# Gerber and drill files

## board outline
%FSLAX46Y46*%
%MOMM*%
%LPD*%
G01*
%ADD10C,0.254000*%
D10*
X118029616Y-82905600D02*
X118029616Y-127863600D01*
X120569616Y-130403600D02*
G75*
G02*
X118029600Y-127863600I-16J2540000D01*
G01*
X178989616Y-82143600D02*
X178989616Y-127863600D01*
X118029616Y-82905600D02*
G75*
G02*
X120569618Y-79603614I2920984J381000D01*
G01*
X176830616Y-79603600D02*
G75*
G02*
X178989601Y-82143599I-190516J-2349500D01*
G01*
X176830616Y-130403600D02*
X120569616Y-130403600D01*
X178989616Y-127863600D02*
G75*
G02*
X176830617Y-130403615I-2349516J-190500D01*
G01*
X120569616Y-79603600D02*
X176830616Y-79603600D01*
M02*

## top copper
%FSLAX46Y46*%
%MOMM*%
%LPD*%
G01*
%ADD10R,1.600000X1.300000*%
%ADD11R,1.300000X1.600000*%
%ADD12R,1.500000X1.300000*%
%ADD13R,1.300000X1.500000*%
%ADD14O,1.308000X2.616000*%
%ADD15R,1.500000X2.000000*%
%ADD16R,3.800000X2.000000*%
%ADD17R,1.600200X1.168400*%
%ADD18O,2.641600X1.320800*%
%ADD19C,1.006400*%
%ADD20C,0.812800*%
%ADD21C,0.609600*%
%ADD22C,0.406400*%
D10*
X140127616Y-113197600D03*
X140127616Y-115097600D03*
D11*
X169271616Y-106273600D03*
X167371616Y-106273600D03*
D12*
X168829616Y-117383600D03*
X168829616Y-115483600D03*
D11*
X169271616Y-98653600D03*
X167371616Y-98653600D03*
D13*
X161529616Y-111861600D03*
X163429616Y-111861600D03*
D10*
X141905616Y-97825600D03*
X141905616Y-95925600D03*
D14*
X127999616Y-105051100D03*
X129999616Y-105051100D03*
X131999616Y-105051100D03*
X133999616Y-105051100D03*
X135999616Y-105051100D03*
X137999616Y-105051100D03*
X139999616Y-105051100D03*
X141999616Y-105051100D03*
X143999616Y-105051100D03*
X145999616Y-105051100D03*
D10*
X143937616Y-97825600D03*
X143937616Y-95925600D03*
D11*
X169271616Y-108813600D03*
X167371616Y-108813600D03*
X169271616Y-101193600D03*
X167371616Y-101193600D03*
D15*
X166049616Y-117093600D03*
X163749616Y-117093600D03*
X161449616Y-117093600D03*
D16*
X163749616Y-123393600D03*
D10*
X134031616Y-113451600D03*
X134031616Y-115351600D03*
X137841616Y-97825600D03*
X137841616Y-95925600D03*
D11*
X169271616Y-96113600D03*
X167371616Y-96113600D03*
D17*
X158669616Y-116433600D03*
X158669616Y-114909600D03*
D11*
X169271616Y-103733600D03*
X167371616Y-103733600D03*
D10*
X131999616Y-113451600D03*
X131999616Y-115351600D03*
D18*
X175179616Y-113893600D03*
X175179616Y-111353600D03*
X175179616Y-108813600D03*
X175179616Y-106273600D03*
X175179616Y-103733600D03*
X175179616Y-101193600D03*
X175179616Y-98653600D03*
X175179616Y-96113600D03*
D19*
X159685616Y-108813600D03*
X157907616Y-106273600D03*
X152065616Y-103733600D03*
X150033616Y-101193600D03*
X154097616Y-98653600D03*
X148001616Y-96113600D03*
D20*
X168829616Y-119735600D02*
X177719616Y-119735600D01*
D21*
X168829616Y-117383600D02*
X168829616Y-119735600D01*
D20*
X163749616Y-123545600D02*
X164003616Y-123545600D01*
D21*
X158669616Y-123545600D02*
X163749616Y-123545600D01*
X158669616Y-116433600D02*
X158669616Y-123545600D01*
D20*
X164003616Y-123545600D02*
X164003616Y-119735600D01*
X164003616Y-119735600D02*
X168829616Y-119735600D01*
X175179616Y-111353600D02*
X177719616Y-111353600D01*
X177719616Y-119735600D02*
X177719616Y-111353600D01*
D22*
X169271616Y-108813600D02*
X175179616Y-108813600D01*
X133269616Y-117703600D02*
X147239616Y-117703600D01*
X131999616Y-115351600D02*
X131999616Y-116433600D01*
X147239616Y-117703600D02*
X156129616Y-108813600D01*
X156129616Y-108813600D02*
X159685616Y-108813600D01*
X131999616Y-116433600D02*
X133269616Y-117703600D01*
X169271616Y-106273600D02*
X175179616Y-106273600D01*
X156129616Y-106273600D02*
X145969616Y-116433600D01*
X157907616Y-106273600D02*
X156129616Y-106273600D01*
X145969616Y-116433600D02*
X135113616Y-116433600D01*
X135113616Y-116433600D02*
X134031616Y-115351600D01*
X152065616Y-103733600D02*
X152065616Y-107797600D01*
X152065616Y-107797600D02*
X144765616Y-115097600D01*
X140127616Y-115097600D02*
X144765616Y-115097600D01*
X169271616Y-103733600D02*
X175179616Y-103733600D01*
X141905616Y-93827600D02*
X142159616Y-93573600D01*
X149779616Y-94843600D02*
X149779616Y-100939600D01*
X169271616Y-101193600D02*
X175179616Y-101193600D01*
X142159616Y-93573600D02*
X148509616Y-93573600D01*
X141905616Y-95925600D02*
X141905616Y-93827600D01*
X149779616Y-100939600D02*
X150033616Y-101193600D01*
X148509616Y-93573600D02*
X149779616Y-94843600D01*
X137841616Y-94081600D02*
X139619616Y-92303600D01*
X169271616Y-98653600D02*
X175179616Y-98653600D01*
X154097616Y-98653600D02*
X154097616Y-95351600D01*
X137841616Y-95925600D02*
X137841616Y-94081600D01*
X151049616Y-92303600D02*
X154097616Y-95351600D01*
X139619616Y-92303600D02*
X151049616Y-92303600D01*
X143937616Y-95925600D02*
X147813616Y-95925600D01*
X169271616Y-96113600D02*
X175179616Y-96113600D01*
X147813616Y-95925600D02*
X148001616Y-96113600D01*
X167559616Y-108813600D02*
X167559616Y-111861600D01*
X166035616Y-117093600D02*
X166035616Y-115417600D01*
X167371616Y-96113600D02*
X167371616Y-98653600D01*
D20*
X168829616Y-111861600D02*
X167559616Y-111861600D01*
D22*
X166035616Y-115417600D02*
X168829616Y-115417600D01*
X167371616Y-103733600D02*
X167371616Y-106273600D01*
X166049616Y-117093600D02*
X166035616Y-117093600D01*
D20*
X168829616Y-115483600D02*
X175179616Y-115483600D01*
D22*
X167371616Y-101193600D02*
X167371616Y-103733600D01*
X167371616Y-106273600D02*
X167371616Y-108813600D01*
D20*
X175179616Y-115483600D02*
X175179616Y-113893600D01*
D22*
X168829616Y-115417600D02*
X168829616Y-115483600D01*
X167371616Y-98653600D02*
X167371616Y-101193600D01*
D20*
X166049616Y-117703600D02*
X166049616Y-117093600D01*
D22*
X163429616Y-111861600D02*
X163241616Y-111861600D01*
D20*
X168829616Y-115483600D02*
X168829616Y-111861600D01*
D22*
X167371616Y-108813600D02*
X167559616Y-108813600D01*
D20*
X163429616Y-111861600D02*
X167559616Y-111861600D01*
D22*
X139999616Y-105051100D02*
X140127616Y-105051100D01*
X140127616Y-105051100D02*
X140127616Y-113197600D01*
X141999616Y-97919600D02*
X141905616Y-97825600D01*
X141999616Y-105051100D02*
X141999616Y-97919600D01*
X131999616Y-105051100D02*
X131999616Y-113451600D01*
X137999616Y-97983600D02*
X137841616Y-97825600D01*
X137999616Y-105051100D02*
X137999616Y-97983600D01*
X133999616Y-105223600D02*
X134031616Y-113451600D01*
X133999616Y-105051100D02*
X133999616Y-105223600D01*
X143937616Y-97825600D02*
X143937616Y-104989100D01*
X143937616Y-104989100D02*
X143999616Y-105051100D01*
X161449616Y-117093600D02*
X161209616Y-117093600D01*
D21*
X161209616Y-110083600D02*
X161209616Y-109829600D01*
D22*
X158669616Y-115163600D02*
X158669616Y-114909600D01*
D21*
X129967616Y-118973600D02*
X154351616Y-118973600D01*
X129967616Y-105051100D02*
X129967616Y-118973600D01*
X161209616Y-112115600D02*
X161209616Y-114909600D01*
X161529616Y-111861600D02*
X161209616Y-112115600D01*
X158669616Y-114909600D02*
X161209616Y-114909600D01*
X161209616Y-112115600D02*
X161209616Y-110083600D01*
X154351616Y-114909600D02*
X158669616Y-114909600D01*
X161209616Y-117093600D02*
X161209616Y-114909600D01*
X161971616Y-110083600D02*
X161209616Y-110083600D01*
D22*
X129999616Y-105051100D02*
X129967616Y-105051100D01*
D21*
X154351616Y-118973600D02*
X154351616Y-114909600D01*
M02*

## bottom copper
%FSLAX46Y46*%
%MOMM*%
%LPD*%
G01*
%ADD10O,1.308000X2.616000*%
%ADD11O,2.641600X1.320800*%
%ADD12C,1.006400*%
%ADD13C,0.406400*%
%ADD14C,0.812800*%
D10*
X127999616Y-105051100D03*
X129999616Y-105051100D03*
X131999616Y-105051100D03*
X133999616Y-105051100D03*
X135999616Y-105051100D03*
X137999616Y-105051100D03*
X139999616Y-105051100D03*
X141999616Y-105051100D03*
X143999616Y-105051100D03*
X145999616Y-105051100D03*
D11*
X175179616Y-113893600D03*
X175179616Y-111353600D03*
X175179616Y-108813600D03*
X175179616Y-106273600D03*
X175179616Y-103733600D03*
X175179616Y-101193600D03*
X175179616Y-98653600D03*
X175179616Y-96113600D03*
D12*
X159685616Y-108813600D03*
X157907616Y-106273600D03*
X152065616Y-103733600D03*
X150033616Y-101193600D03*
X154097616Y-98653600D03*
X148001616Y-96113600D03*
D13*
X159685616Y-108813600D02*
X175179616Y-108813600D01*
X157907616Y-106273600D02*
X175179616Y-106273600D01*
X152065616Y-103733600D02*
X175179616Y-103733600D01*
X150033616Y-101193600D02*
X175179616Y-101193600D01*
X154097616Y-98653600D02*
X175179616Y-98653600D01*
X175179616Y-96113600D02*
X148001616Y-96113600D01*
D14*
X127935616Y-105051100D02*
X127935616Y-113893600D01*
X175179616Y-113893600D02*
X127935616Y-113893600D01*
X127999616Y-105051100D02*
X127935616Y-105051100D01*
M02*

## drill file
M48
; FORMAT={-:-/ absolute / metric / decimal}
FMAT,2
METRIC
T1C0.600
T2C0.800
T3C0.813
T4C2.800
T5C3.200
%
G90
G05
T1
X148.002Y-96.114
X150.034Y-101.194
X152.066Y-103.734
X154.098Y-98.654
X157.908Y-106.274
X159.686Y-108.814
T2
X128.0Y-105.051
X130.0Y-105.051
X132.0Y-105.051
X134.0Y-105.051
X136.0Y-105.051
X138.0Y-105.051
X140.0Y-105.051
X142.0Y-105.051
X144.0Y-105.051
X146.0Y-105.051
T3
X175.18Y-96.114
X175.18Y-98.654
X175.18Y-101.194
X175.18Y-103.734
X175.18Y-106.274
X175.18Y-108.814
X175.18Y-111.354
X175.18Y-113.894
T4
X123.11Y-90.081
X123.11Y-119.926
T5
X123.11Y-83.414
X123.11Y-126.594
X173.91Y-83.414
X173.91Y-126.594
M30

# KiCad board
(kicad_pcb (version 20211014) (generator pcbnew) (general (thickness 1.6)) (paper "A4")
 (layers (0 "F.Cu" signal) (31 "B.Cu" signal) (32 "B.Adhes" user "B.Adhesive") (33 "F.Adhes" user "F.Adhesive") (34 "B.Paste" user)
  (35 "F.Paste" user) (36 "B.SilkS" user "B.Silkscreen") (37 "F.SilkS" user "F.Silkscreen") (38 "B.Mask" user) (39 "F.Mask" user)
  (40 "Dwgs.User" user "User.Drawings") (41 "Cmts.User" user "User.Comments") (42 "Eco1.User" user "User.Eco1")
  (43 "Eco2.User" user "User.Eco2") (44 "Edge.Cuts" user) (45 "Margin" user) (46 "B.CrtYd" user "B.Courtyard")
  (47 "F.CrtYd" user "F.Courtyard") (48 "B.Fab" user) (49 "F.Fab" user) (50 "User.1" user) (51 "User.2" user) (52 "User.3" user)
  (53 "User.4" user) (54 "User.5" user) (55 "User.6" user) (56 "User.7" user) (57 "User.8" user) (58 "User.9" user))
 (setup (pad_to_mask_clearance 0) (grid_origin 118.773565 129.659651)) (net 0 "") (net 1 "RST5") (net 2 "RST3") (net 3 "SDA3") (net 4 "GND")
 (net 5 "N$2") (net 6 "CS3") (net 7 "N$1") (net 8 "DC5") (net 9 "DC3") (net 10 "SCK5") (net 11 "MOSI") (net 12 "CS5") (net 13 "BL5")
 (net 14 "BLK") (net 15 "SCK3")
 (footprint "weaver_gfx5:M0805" (layer "F.Cu") (at 140.127616 114.1476 -90)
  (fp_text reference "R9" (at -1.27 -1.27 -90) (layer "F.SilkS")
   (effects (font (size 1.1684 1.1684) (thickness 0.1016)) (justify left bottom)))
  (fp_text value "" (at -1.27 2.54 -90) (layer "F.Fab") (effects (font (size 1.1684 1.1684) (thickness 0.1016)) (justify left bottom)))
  (pad "1" smd rect (at -0.95 0 270) (size 1.3 1.6) (layers "F.Cu" "F.Paste" "F.Mask") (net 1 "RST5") (solder_mask_margin 0.1016))
  (pad "2" smd rect (at 0.95 0 270) (size 1.3 1.6) (layers "F.Cu" "F.Paste" "F.Mask") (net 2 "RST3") (solder_mask_margin 0.1016)))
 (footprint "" (layer "F.Cu") (at 173.909616 83.4136)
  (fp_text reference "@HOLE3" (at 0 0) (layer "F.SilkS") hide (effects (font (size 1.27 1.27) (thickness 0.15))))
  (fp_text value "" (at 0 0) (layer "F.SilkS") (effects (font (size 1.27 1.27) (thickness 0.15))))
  (pad "" np_thru_hole circle (at 0 0) (size 3.2 3.2) (drill 3.2) (layers *.Cu *.Mask)))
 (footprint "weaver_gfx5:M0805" (layer "F.Cu") (at 168.321616 106.2736 180)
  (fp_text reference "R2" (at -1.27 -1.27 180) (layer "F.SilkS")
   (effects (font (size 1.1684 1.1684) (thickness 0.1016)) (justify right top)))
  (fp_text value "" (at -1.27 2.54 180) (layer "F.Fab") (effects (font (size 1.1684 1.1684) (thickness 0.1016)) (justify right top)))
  (pad "1" smd rect (at -0.95 0 180) (size 1.3 1.6) (layers "F.Cu" "F.Paste" "F.Mask") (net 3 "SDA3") (solder_mask_margin 0.1016))
  (pad "2" smd rect (at 0.95 0 180) (size 1.3 1.6) (layers "F.Cu" "F.Paste" "F.Mask") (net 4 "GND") (solder_mask_margin 0.1016)))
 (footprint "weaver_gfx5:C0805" (layer "F.Cu") (at 168.829616 116.4336 90)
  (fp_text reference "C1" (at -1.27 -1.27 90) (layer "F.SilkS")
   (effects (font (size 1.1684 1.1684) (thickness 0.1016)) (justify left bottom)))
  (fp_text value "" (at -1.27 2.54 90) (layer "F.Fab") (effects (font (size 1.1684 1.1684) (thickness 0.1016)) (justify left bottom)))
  (pad "1" smd rect (at -0.95 0 90) (size 1.3 1.5) (layers "F.Cu" "F.Paste" "F.Mask") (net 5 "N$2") (solder_mask_margin 0.1016))
  (pad "2" smd rect (at 0.95 0 90) (size 1.3 1.5) (layers "F.Cu" "F.Paste" "F.Mask") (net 4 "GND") (solder_mask_margin 0.1016)))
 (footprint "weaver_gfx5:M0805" (layer "F.Cu") (at 168.321616 98.6536 180)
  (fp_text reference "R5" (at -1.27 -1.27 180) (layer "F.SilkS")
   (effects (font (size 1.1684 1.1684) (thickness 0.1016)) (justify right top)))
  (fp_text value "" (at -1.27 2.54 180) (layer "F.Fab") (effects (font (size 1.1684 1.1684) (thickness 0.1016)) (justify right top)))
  (pad "1" smd rect (at -0.95 0 180) (size 1.3 1.6) (layers "F.Cu" "F.Paste" "F.Mask") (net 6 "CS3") (solder_mask_margin 0.1016))
  (pad "2" smd rect (at 0.95 0 180) (size 1.3 1.6) (layers "F.Cu" "F.Paste" "F.Mask") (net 4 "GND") (solder_mask_margin 0.1016)))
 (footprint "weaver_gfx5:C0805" (layer "F.Cu") (at 162.479616 111.8616)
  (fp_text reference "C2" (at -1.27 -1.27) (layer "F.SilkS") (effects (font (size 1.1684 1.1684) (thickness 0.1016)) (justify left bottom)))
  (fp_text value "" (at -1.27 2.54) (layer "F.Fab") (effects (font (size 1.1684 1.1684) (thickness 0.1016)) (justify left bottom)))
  (pad "1" smd rect (at -0.95 0) (size 1.3 1.5) (layers "F.Cu" "F.Paste" "F.Mask") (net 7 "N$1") (solder_mask_margin 0.1016))
  (pad "2" smd rect (at 0.95 0) (size 1.3 1.5) (layers "F.Cu" "F.Paste" "F.Mask") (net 4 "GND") (solder_mask_margin 0.1016)))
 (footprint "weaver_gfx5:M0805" (layer "F.Cu") (at 141.905616 96.8756 90)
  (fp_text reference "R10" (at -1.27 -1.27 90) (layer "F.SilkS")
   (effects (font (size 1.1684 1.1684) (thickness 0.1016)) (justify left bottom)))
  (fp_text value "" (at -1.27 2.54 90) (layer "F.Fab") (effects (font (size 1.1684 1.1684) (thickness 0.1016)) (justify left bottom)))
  (pad "1" smd rect (at -0.95 0 90) (size 1.3 1.6) (layers "F.Cu" "F.Paste" "F.Mask") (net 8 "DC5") (solder_mask_margin 0.1016))
  (pad "2" smd rect (at 0.95 0 90) (size 1.3 1.6) (layers "F.Cu" "F.Paste" "F.Mask") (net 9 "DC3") (solder_mask_margin 0.1016)))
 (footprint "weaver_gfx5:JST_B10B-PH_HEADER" (layer "F.Cu") (at 131.999616 105.0036 180)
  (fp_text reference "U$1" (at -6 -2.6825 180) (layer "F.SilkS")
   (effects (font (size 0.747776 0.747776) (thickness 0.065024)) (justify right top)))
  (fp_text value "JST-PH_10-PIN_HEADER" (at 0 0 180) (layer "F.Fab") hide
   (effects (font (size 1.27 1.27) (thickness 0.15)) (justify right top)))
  (pad "P1" thru_hole oval (at 4 -0.0475 270) (size 2.616 1.308) (drill 0.8) (layers *.Cu *.Mask) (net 4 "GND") (solder_mask_margin 0.1016))
  (pad "P2" thru_hole oval (at 2 -0.0475 270) (size 2.616 1.308) (drill 0.8) (layers *.Cu *.Mask) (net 7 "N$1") (solder_mask_margin 0.1016))
  (pad "P3" thru_hole oval (at 0 -0.0475 270) (size 2.616 1.308) (drill 0.8) (layers *.Cu *.Mask) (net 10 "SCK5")
   (solder_mask_margin 0.1016))
  (pad "P4" thru_hole oval (at -2 -0.0475 270) (size 2.616 1.308) (drill 0.8) (layers *.Cu *.Mask) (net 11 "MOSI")
   (solder_mask_margin 0.1016))
  (pad "P5" thru_hole oval (at -4 -0.0475 270) (size 2.616 1.308) (drill 0.8) (layers *.Cu *.Mask) (solder_mask_margin 0.1016))
  (pad "P6" thru_hole oval (at -6 -0.0475 270) (size 2.616 1.308) (drill 0.8) (layers *.Cu *.Mask) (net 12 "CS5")
   (solder_mask_margin 0.1016))
  (pad "P7" thru_hole oval (at -8 -0.0475 270) (size 2.616 1.308) (drill 0.8) (layers *.Cu *.Mask) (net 1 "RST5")
   (solder_mask_margin 0.1016))
  (pad "P8" thru_hole oval (at -10 -0.0475 270) (size 2.616 1.308) (drill 0.8) (layers *.Cu *.Mask) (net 8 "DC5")
   (solder_mask_margin 0.1016))
  (pad "P9" thru_hole oval (at -12 -0.0475 270) (size 2.616 1.308) (drill 0.8) (layers *.Cu *.Mask) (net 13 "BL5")
   (solder_mask_margin 0.1016))
  (pad "P10" thru_hole oval (at -14 -0.0475 270) (size 2.616 1.308) (drill 0.8) (layers *.Cu *.Mask) (solder_mask_margin 0.1016)))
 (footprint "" (layer "F.Cu") (at 123.109616 83.4136)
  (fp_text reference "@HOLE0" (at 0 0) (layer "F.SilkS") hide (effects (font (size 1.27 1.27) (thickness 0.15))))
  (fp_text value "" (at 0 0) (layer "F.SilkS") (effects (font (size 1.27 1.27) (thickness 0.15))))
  (pad "" np_thru_hole circle (at 0 0) (size 3.2 3.2) (drill 3.2) (layers *.Cu *.Mask)))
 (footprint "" (layer "F.Cu") (at 123.109616 90.0811)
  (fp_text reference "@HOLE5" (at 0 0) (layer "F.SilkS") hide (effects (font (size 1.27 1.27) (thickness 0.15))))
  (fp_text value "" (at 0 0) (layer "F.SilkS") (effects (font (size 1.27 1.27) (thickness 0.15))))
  (pad "" np_thru_hole circle (at 0 0) (size 2.8 2.8) (drill 2.8) (layers *.Cu *.Mask)))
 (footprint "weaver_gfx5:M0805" (layer "F.Cu") (at 143.937616 96.8756 90)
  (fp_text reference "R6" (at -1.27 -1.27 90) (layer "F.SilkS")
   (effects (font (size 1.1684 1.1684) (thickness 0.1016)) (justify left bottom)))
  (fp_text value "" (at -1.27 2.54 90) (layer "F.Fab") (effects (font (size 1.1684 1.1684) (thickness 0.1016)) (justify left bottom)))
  (pad "1" smd rect (at -0.95 0 90) (size 1.3 1.6) (layers "F.Cu" "F.Paste" "F.Mask") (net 13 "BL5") (solder_mask_margin 0.1016))
  (pad "2" smd rect (at 0.95 0 90) (size 1.3 1.6) (layers "F.Cu" "F.Paste" "F.Mask") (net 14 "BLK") (solder_mask_margin 0.1016)))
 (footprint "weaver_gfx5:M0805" (layer "F.Cu") (at 168.321616 108.8136 180)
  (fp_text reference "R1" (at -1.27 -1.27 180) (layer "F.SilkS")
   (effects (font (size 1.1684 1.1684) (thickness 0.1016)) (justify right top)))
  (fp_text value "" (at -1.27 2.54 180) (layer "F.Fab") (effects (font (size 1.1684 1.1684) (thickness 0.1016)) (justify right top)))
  (pad "1" smd rect (at -0.95 0 180) (size 1.3 1.6) (layers "F.Cu" "F.Paste" "F.Mask") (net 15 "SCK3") (solder_mask_margin 0.1016))
  (pad "2" smd rect (at 0.95 0 180) (size 1.3 1.6) (layers "F.Cu" "F.Paste" "F.Mask") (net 4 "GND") (solder_mask_margin 0.1016)))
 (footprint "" (layer "F.Cu") (at 123.109616 119.9261)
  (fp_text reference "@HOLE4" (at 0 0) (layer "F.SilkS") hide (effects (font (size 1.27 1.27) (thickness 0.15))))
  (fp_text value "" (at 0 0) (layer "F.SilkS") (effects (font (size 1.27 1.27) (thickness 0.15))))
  (pad "" np_thru_hole circle (at 0 0) (size 2.8 2.8) (drill 2.8) (layers *.Cu *.Mask)))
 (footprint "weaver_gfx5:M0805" (layer "F.Cu") (at 168.321616 101.1936 180)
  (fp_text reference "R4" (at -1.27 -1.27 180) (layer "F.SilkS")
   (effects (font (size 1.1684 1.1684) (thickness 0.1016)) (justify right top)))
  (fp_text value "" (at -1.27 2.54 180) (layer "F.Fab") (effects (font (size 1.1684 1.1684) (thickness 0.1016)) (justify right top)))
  (pad "1" smd rect (at -0.95 0 180) (size 1.3 1.6) (layers "F.Cu" "F.Paste" "F.Mask") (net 9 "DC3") (solder_mask_margin 0.1016))
  (pad "2" smd rect (at 0.95 0 180) (size 1.3 1.6) (layers "F.Cu" "F.Paste" "F.Mask") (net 4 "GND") (solder_mask_margin 0.1016)))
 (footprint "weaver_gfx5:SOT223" (layer "F.Cu") (at 163.749616 120.2436 180)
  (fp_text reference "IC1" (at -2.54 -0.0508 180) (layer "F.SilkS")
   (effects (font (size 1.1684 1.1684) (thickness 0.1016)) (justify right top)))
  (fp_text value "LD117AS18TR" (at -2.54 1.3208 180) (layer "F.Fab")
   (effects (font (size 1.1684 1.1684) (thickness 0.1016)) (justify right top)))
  (pad "1" smd rect (at -2.3 3.15 180) (size 1.5 2) (layers "F.Cu" "F.Paste" "F.Mask") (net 4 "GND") (solder_mask_margin 0.1016))
  (pad "2" smd rect (at 0 3.15 180) (size 1.5 2) (layers "F.Cu" "F.Paste" "F.Mask") (solder_mask_margin 0.1016))
  (pad "3" smd rect (at 2.3 3.15 180) (size 1.5 2) (layers "F.Cu" "F.Paste" "F.Mask") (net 7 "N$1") (solder_mask_margin 0.1016))
  (pad "4" smd rect (at 0 -3.15 180) (size 3.8 2) (layers "F.Cu" "F.Paste" "F.Mask") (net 5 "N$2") (solder_mask_margin 0.1016)))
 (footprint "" (layer "F.Cu") (at 123.109616 126.5936)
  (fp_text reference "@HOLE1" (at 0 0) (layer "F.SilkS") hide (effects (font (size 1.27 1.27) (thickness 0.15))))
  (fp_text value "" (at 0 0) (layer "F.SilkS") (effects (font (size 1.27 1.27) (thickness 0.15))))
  (pad "" np_thru_hole circle (at 0 0) (size 3.2 3.2) (drill 3.2) (layers *.Cu *.Mask)))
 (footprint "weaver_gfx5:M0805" (layer "F.Cu") (at 134.031616 114.4016 -90)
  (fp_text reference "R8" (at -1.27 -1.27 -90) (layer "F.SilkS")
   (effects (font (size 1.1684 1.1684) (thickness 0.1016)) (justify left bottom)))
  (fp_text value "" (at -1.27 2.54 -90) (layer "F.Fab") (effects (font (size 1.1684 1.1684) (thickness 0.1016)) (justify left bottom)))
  (pad "1" smd rect (at -0.95 0 270) (size 1.3 1.6) (layers "F.Cu" "F.Paste" "F.Mask") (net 11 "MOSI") (solder_mask_margin 0.1016))
  (pad "2" smd rect (at 0.95 0 270) (size 1.3 1.6) (layers "F.Cu" "F.Paste" "F.Mask") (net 3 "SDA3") (solder_mask_margin 0.1016)))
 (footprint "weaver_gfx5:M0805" (layer "F.Cu") (at 137.841616 96.8756 90)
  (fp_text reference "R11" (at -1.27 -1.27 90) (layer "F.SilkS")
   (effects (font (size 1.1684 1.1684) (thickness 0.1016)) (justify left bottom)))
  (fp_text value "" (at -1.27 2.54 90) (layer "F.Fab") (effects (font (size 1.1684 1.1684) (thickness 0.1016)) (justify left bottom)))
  (pad "1" smd rect (at -0.95 0 90) (size 1.3 1.6) (layers "F.Cu" "F.Paste" "F.Mask") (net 12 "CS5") (solder_mask_margin 0.1016))
  (pad "2" smd rect (at 0.95 0 90) (size 1.3 1.6) (layers "F.Cu" "F.Paste" "F.Mask") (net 6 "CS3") (solder_mask_margin 0.1016)))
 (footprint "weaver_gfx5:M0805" (layer "F.Cu") (at 168.321616 96.1136 180)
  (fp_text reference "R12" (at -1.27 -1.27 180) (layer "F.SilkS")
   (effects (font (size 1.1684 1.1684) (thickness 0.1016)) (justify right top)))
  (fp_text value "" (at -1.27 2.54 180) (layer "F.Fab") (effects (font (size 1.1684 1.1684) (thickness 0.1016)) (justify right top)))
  (pad "1" smd rect (at -0.95 0 180) (size 1.3 1.6) (layers "F.Cu" "F.Paste" "F.Mask") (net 14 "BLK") (solder_mask_margin 0.1016))
  (pad "2" smd rect (at 0.95 0 180) (size 1.3 1.6) (layers "F.Cu" "F.Paste" "F.Mask") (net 4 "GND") (solder_mask_margin 0.1016)))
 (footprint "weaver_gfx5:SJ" (layer "F.Cu") (at 158.669616 115.6716 90)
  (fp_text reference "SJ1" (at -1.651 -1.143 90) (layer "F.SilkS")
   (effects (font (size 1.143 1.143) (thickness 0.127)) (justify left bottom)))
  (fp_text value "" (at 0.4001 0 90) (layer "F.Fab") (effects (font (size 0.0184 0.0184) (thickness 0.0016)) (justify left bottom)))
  (pad "1" smd rect (at -0.762 0 90) (size 1.1684 1.6002) (layers "F.Cu" "F.Paste" "F.Mask") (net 5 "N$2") (solder_mask_margin 0.1016))
  (pad "2" smd rect (at 0.762 0 90) (size 1.1684 1.6002) (layers "F.Cu" "F.Paste" "F.Mask") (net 7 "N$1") (solder_mask_margin 0.1016)))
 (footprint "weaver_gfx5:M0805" (layer "F.Cu") (at 168.321616 103.7336 180)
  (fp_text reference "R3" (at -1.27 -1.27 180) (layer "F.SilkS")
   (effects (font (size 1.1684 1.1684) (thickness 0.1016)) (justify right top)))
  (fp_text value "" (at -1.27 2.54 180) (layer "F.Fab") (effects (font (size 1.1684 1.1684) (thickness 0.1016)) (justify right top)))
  (pad "1" smd rect (at -0.95 0 180) (size 1.3 1.6) (layers "F.Cu" "F.Paste" "F.Mask") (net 2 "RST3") (solder_mask_margin 0.1016))
  (pad "2" smd rect (at 0.95 0 180) (size 1.3 1.6) (layers "F.Cu" "F.Paste" "F.Mask") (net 4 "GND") (solder_mask_margin 0.1016)))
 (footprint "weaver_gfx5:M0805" (layer "F.Cu") (at 131.999616 114.4016 -90)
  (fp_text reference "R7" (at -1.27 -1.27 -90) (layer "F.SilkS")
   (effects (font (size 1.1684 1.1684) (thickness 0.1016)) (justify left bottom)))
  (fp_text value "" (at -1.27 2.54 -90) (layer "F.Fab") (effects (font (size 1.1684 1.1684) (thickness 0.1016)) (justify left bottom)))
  (pad "1" smd rect (at -0.95 0 270) (size 1.3 1.6) (layers "F.Cu" "F.Paste" "F.Mask") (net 10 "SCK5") (solder_mask_margin 0.1016))
  (pad "2" smd rect (at 0.95 0 270) (size 1.3 1.6) (layers "F.Cu" "F.Paste" "F.Mask") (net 15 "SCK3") (solder_mask_margin 0.1016)))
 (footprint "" (layer "F.Cu") (at 173.909616 126.5936)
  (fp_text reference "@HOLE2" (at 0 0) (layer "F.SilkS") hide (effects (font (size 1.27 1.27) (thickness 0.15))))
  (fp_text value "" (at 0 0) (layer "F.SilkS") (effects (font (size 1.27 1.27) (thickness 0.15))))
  (pad "" np_thru_hole circle (at 0 0) (size 3.2 3.2) (drill 3.2) (layers *.Cu *.Mask)))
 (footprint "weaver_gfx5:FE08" (layer "B.Cu") (at 175.179616 105.0036 90)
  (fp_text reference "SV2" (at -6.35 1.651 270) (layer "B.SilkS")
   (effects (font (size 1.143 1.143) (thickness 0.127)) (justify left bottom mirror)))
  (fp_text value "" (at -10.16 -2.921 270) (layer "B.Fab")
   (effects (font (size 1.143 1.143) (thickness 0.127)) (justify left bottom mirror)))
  (pad "1" thru_hole oval (at -8.89 0) (size 2.6416 1.3208) (drill 0.8128) (layers *.Cu *.Mask) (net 4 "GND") (solder_mask_margin 0.1016))
  (pad "2" thru_hole oval (at -6.35 0) (size 2.6416 1.3208) (drill 0.8128) (layers *.Cu *.Mask) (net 5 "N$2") (solder_mask_margin 0.1016))
  (pad "3" thru_hole oval (at -3.81 0) (size 2.6416 1.3208) (drill 0.8128) (layers *.Cu *.Mask) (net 15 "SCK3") (solder_mask_margin 0.1016))
  (pad "4" thru_hole oval (at -1.27 0) (size 2.6416 1.3208) (drill 0.8128) (layers *.Cu *.Mask) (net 3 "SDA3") (solder_mask_margin 0.1016))
  (pad "5" thru_hole oval (at 1.27 0) (size 2.6416 1.3208) (drill 0.8128) (layers *.Cu *.Mask) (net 2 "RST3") (solder_mask_margin 0.1016))
  (pad "6" thru_hole oval (at 3.81 0) (size 2.6416 1.3208) (drill 0.8128) (layers *.Cu *.Mask) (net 9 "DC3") (solder_mask_margin 0.1016))
  (pad "7" thru_hole oval (at 6.35 0) (size 2.6416 1.3208) (drill 0.8128) (layers *.Cu *.Mask) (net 6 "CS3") (solder_mask_margin 0.1016))
  (pad "8" thru_hole oval (at 8.89 0) (size 2.6416 1.3208) (drill 0.8128) (layers *.Cu *.Mask) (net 14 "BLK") (solder_mask_margin 0.1016)))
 (gr_line (start 118.029616 82.9056) (end 118.029616 127.8636) (layer "Edge.Cuts") (width 0.254))
 (gr_arc (start 120.569616 130.4036) (mid 118.773565 129.659651) (end 118.029616 127.8636) (layer "Edge.Cuts") (width 0.254))
 (gr_line (start 178.989616 82.1436) (end 178.989616 127.8636) (layer "Edge.Cuts") (width 0.254))
 (gr_arc (start 118.029616 82.9056) (mid 118.615749 80.728549) (end 120.569616 79.6036) (layer "Edge.Cuts") (width 0.254))
 (gr_arc (start 176.830616 79.6036) (mid 178.436167 80.426456) (end 178.989616 82.1436) (layer "Edge.Cuts") (width 0.254))
 (gr_line (start 176.830616 130.4036) (end 120.569616 130.4036) (layer "Edge.Cuts") (width 0.254))
 (gr_arc (start 178.989616 127.8636) (mid 178.436167 129.580744) (end 176.830616 130.4036) (layer "Edge.Cuts") (width 0.254))
 (gr_line (start 120.569616 79.6036) (end 176.830616 79.6036) (layer "Edge.Cuts") (width 0.254))
 (segment (start 168.829616 119.7356) (end 177.719616 119.7356) (width 0.8128) (layer "F.Cu") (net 5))
 (segment (start 168.829616 117.3836) (end 168.829616 119.7356) (width 0.6096) (layer "F.Cu") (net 5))
 (segment (start 163.749616 123.5456) (end 164.003616 123.5456) (width 0.8128) (layer "F.Cu") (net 5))
 (segment (start 158.669616 123.5456) (end 163.749616 123.5456) (width 0.6096) (layer "F.Cu") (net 5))
 (segment (start 158.669616 116.4336) (end 158.669616 123.5456) (width 0.6096) (layer "F.Cu") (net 5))
 (segment (start 164.003616 123.5456) (end 164.003616 119.7356) (width 0.8128) (layer "F.Cu") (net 5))
 (segment (start 164.003616 119.7356) (end 168.829616 119.7356) (width 0.8128) (layer "F.Cu") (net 5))
 (segment (start 175.179616 111.3536) (end 177.719616 111.3536) (width 0.8128) (layer "F.Cu") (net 5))
 (segment (start 177.719616 119.7356) (end 177.719616 111.3536) (width 0.8128) (layer "F.Cu") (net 5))
 (segment (start 169.271616 108.8136) (end 175.179616 108.8136) (width 0.4064) (layer "F.Cu") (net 15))
 (segment (start 133.269616 117.7036) (end 147.239616 117.7036) (width 0.4064) (layer "F.Cu") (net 15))
 (segment (start 131.999616 115.3516) (end 131.999616 116.4336) (width 0.4064) (layer "F.Cu") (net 15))
 (segment (start 147.239616 117.7036) (end 156.129616 108.8136) (width 0.4064) (layer "F.Cu") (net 15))
 (segment (start 156.129616 108.8136) (end 159.685616 108.8136) (width 0.4064) (layer "F.Cu") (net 15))
 (segment (start 131.999616 116.4336) (end 133.269616 117.7036) (width 0.4064) (layer "F.Cu") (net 15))
 (via (at 159.685616 108.8136) (size 1.0064) (drill 0.6) (layers "F.Cu" "B.Cu") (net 15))
 (segment (start 159.685616 108.8136) (end 175.179616 108.8136) (width 0.4064) (layer "B.Cu") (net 15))
 (segment (start 169.271616 106.2736) (end 175.179616 106.2736) (width 0.4064) (layer "F.Cu") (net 3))
 (segment (start 156.129616 106.2736) (end 145.969616 116.4336) (width 0.4064) (layer "F.Cu") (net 3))
 (segment (start 157.907616 106.2736) (end 156.129616 106.2736) (width 0.4064) (layer "F.Cu") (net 3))
 (segment (start 145.969616 116.4336) (end 135.113616 116.4336) (width 0.4064) (layer "F.Cu") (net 3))
 (segment (start 135.113616 116.4336) (end 134.031616 115.3516) (width 0.4064) (layer "F.Cu") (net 3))
 (via (at 157.907616 106.2736) (size 1.0064) (drill 0.6) (layers "F.Cu" "B.Cu") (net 3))
 (segment (start 157.907616 106.2736) (end 175.179616 106.2736) (width 0.4064) (layer "B.Cu") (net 3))
 (segment (start 152.065616 103.7336) (end 152.065616 107.7976) (width 0.4064) (layer "F.Cu") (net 2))
 (segment (start 152.065616 107.7976) (end 144.765616 115.0976) (width 0.4064) (layer "F.Cu") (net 2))
 (segment (start 140.127616 115.0976) (end 144.765616 115.0976) (width 0.4064) (layer "F.Cu") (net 2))
 (segment (start 169.271616 103.7336) (end 175.179616 103.7336) (width 0.4064) (layer "F.Cu") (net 2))
 (via (at 152.065616 103.7336) (size 1.0064) (drill 0.6) (layers "F.Cu" "B.Cu") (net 2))
 (segment (start 152.065616 103.7336) (end 175.179616 103.7336) (width 0.4064) (layer "B.Cu") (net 2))
 (segment (start 141.905616 93.8276) (end 142.159616 93.5736) (width 0.4064) (layer "F.Cu") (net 9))
 (segment (start 149.779616 94.8436) (end 149.779616 100.9396) (width 0.4064) (layer "F.Cu") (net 9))
 (segment (start 169.271616 101.1936) (end 175.179616 101.1936) (width 0.4064) (layer "F.Cu") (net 9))
 (segment (start 142.159616 93.5736) (end 148.509616 93.5736) (width 0.4064) (layer "F.Cu") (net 9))
 (segment (start 141.905616 95.9256) (end 141.905616 93.8276) (width 0.4064) (layer "F.Cu") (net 9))
 (segment (start 149.779616 100.9396) (end 150.033616 101.1936) (width 0.4064) (layer "F.Cu") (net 9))
 (segment (start 148.509616 93.5736) (end 149.779616 94.8436) (width 0.4064) (layer "F.Cu") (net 9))
 (via (at 150.033616 101.1936) (size 1.0064) (drill 0.6) (layers "F.Cu" "B.Cu") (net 9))
 (segment (start 150.033616 101.1936) (end 175.179616 101.1936) (width 0.4064) (layer "B.Cu") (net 9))
 (segment (start 137.841616 94.0816) (end 139.619616 92.3036) (width 0.4064) (layer "F.Cu") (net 6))
 (segment (start 169.271616 98.6536) (end 175.179616 98.6536) (width 0.4064) (layer "F.Cu") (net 6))
 (segment (start 154.097616 98.6536) (end 154.097616 95.3516) (width 0.4064) (layer "F.Cu") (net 6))
 (segment (start 137.841616 95.9256) (end 137.841616 94.0816) (width 0.4064) (layer "F.Cu") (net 6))
 (segment (start 151.049616 92.3036) (end 154.097616 95.3516) (width 0.4064) (layer "F.Cu") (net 6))
 (segment (start 139.619616 92.3036) (end 151.049616 92.3036) (width 0.4064) (layer "F.Cu") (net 6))
 (via (at 154.097616 98.6536) (size 1.0064) (drill 0.6) (layers "F.Cu" "B.Cu") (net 6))
 (segment (start 154.097616 98.6536) (end 175.179616 98.6536) (width 0.4064) (layer "B.Cu") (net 6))
 (segment (start 143.937616 95.9256) (end 147.813616 95.9256) (width 0.4064) (layer "F.Cu") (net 14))
 (segment (start 169.271616 96.1136) (end 175.179616 96.1136) (width 0.4064) (layer "F.Cu") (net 14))
 (segment (start 147.813616 95.9256) (end 148.001616 96.1136) (width 0.4064) (layer "F.Cu") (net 14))
 (via (at 148.001616 96.1136) (size 1.0064) (drill 0.6) (layers "F.Cu" "B.Cu") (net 14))
 (segment (start 175.179616 96.1136) (end 148.001616 96.1136) (width 0.4064) (layer "B.Cu") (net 14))
 (segment (start 167.559616 108.8136) (end 167.559616 111.8616) (width 0.4064) (layer "F.Cu") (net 4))
 (segment (start 166.035616 117.0936) (end 166.035616 115.4176) (width 0.4064) (layer "F.Cu") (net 4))
 (segment (start 167.371616 96.1136) (end 167.371616 98.6536) (width 0.4064) (layer "F.Cu") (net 4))
 (segment (start 168.829616 111.8616) (end 167.559616 111.8616) (width 0.8128) (layer "F.Cu") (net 4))
 (segment (start 166.035616 115.4176) (end 168.829616 115.4176) (width 0.4064) (layer "F.Cu") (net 4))
 (segment (start 167.371616 103.7336) (end 167.371616 106.2736) (width 0.4064) (layer "F.Cu") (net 4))
 (segment (start 166.049616 117.0936) (end 166.035616 117.0936) (width 0.4064) (layer "F.Cu") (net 4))
 (segment (start 168.829616 115.4836) (end 175.179616 115.4836) (width 0.8128) (layer "F.Cu") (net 4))
 (segment (start 167.371616 101.1936) (end 167.371616 103.7336) (width 0.4064) (layer "F.Cu") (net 4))
 (segment (start 167.371616 106.2736) (end 167.371616 108.8136) (width 0.4064) (layer "F.Cu") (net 4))
 (segment (start 175.179616 115.4836) (end 175.179616 113.8936) (width 0.8128) (layer "F.Cu") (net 4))
 (segment (start 168.829616 115.4176) (end 168.829616 115.4836) (width 0.4064) (layer "F.Cu") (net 4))
 (segment (start 167.371616 98.6536) (end 167.371616 101.1936) (width 0.4064) (layer "F.Cu") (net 4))
 (segment (start 166.049616 117.7036) (end 166.049616 117.0936) (width 0.8128) (layer "F.Cu") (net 4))
 (segment (start 163.429616 111.8616) (end 163.241616 111.8616) (width 0.4064) (layer "F.Cu") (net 4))
 (segment (start 168.829616 115.4836) (end 168.829616 111.8616) (width 0.8128) (layer "F.Cu") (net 4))
 (segment (start 167.371616 108.8136) (end 167.559616 108.8136) (width 0.4064) (layer "F.Cu") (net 4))
 (segment (start 163.429616 111.8616) (end 167.559616 111.8616) (width 0.8128) (layer "F.Cu") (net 4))
 (segment (start 127.935616 105.0511) (end 127.935616 113.8936) (width 0.8128) (layer "B.Cu") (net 4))
 (segment (start 175.179616 113.8936) (end 127.935616 113.8936) (width 0.8128) (layer "B.Cu") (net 4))
 (segment (start 127.999616 105.0511) (end 127.935616 105.0511) (width 0.8128) (layer "B.Cu") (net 4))
 (segment (start 139.999616 105.0511) (end 140.127616 105.0511) (width 0.4064) (layer "F.Cu") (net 1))
 (segment (start 140.127616 105.0511) (end 140.127616 113.1976) (width 0.4064) (layer "F.Cu") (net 1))
 (segment (start 141.999616 97.9196) (end 141.905616 97.8256) (width 0.4064) (layer "F.Cu") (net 8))
 (segment (start 141.999616 105.0511) (end 141.999616 97.9196) (width 0.4064) (layer "F.Cu") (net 8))
 (segment (start 131.999616 105.0511) (end 131.999616 113.4516) (width 0.4064) (layer "F.Cu") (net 10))
 (segment (start 137.999616 97.9836) (end 137.841616 97.8256) (width 0.4064) (layer "F.Cu") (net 12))
 (segment (start 137.999616 105.0511) (end 137.999616 97.9836) (width 0.4064) (layer "F.Cu") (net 12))
 (segment (start 133.999616 105.2236) (end 134.031616 113.4516) (width 0.4064) (layer "F.Cu") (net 11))
 (segment (start 133.999616 105.0511) (end 133.999616 105.2236) (width 0.4064) (layer "F.Cu") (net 11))
 (segment (start 143.937616 97.8256) (end 143.937616 104.9891) (width 0.4064) (layer "F.Cu") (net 13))
 (segment (start 143.937616 104.9891) (end 143.999616 105.0511) (width 0.4064) (layer "F.Cu") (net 13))
 (segment (start 161.449616 117.0936) (end 161.209616 117.0936) (width 0.4064) (layer "F.Cu") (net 7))
 (segment (start 161.209616 110.0836) (end 161.209616 109.8296) (width 0.6096) (layer "F.Cu") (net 7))
 (segment (start 158.669616 115.1636) (end 158.669616 114.9096) (width 0.4064) (layer "F.Cu") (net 7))
 (segment (start 129.967616 118.9736) (end 154.351616 118.9736) (width 0.6096) (layer "F.Cu") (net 7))
 (segment (start 129.967616 105.0511) (end 129.967616 118.9736) (width 0.6096) (layer "F.Cu") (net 7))
 (segment (start 161.209616 112.1156) (end 161.209616 114.9096) (width 0.6096) (layer "F.Cu") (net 7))
 (segment (start 161.529616 111.8616) (end 161.209616 112.1156) (width 0.6096) (layer "F.Cu") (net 7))
 (segment (start 158.669616 114.9096) (end 161.209616 114.9096) (width 0.6096) (layer "F.Cu") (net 7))
 (segment (start 161.209616 112.1156) (end 161.209616 110.0836) (width 0.6096) (layer "F.Cu") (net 7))
 (segment (start 154.351616 114.9096) (end 158.669616 114.9096) (width 0.6096) (layer "F.Cu") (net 7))
 (segment (start 161.209616 117.0936) (end 161.209616 114.9096) (width 0.6096) (layer "F.Cu") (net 7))
 (segment (start 161.971616 110.0836) (end 161.209616 110.0836) (width 0.6096) (layer "F.Cu") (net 7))
 (segment (start 129.999616 105.0511) (end 129.967616 105.0511) (width 0.4064) (layer "F.Cu") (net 7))
 (segment (start 154.351616 118.9736) (end 154.351616 114.9096) (width 0.6096) (layer "F.Cu") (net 7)))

